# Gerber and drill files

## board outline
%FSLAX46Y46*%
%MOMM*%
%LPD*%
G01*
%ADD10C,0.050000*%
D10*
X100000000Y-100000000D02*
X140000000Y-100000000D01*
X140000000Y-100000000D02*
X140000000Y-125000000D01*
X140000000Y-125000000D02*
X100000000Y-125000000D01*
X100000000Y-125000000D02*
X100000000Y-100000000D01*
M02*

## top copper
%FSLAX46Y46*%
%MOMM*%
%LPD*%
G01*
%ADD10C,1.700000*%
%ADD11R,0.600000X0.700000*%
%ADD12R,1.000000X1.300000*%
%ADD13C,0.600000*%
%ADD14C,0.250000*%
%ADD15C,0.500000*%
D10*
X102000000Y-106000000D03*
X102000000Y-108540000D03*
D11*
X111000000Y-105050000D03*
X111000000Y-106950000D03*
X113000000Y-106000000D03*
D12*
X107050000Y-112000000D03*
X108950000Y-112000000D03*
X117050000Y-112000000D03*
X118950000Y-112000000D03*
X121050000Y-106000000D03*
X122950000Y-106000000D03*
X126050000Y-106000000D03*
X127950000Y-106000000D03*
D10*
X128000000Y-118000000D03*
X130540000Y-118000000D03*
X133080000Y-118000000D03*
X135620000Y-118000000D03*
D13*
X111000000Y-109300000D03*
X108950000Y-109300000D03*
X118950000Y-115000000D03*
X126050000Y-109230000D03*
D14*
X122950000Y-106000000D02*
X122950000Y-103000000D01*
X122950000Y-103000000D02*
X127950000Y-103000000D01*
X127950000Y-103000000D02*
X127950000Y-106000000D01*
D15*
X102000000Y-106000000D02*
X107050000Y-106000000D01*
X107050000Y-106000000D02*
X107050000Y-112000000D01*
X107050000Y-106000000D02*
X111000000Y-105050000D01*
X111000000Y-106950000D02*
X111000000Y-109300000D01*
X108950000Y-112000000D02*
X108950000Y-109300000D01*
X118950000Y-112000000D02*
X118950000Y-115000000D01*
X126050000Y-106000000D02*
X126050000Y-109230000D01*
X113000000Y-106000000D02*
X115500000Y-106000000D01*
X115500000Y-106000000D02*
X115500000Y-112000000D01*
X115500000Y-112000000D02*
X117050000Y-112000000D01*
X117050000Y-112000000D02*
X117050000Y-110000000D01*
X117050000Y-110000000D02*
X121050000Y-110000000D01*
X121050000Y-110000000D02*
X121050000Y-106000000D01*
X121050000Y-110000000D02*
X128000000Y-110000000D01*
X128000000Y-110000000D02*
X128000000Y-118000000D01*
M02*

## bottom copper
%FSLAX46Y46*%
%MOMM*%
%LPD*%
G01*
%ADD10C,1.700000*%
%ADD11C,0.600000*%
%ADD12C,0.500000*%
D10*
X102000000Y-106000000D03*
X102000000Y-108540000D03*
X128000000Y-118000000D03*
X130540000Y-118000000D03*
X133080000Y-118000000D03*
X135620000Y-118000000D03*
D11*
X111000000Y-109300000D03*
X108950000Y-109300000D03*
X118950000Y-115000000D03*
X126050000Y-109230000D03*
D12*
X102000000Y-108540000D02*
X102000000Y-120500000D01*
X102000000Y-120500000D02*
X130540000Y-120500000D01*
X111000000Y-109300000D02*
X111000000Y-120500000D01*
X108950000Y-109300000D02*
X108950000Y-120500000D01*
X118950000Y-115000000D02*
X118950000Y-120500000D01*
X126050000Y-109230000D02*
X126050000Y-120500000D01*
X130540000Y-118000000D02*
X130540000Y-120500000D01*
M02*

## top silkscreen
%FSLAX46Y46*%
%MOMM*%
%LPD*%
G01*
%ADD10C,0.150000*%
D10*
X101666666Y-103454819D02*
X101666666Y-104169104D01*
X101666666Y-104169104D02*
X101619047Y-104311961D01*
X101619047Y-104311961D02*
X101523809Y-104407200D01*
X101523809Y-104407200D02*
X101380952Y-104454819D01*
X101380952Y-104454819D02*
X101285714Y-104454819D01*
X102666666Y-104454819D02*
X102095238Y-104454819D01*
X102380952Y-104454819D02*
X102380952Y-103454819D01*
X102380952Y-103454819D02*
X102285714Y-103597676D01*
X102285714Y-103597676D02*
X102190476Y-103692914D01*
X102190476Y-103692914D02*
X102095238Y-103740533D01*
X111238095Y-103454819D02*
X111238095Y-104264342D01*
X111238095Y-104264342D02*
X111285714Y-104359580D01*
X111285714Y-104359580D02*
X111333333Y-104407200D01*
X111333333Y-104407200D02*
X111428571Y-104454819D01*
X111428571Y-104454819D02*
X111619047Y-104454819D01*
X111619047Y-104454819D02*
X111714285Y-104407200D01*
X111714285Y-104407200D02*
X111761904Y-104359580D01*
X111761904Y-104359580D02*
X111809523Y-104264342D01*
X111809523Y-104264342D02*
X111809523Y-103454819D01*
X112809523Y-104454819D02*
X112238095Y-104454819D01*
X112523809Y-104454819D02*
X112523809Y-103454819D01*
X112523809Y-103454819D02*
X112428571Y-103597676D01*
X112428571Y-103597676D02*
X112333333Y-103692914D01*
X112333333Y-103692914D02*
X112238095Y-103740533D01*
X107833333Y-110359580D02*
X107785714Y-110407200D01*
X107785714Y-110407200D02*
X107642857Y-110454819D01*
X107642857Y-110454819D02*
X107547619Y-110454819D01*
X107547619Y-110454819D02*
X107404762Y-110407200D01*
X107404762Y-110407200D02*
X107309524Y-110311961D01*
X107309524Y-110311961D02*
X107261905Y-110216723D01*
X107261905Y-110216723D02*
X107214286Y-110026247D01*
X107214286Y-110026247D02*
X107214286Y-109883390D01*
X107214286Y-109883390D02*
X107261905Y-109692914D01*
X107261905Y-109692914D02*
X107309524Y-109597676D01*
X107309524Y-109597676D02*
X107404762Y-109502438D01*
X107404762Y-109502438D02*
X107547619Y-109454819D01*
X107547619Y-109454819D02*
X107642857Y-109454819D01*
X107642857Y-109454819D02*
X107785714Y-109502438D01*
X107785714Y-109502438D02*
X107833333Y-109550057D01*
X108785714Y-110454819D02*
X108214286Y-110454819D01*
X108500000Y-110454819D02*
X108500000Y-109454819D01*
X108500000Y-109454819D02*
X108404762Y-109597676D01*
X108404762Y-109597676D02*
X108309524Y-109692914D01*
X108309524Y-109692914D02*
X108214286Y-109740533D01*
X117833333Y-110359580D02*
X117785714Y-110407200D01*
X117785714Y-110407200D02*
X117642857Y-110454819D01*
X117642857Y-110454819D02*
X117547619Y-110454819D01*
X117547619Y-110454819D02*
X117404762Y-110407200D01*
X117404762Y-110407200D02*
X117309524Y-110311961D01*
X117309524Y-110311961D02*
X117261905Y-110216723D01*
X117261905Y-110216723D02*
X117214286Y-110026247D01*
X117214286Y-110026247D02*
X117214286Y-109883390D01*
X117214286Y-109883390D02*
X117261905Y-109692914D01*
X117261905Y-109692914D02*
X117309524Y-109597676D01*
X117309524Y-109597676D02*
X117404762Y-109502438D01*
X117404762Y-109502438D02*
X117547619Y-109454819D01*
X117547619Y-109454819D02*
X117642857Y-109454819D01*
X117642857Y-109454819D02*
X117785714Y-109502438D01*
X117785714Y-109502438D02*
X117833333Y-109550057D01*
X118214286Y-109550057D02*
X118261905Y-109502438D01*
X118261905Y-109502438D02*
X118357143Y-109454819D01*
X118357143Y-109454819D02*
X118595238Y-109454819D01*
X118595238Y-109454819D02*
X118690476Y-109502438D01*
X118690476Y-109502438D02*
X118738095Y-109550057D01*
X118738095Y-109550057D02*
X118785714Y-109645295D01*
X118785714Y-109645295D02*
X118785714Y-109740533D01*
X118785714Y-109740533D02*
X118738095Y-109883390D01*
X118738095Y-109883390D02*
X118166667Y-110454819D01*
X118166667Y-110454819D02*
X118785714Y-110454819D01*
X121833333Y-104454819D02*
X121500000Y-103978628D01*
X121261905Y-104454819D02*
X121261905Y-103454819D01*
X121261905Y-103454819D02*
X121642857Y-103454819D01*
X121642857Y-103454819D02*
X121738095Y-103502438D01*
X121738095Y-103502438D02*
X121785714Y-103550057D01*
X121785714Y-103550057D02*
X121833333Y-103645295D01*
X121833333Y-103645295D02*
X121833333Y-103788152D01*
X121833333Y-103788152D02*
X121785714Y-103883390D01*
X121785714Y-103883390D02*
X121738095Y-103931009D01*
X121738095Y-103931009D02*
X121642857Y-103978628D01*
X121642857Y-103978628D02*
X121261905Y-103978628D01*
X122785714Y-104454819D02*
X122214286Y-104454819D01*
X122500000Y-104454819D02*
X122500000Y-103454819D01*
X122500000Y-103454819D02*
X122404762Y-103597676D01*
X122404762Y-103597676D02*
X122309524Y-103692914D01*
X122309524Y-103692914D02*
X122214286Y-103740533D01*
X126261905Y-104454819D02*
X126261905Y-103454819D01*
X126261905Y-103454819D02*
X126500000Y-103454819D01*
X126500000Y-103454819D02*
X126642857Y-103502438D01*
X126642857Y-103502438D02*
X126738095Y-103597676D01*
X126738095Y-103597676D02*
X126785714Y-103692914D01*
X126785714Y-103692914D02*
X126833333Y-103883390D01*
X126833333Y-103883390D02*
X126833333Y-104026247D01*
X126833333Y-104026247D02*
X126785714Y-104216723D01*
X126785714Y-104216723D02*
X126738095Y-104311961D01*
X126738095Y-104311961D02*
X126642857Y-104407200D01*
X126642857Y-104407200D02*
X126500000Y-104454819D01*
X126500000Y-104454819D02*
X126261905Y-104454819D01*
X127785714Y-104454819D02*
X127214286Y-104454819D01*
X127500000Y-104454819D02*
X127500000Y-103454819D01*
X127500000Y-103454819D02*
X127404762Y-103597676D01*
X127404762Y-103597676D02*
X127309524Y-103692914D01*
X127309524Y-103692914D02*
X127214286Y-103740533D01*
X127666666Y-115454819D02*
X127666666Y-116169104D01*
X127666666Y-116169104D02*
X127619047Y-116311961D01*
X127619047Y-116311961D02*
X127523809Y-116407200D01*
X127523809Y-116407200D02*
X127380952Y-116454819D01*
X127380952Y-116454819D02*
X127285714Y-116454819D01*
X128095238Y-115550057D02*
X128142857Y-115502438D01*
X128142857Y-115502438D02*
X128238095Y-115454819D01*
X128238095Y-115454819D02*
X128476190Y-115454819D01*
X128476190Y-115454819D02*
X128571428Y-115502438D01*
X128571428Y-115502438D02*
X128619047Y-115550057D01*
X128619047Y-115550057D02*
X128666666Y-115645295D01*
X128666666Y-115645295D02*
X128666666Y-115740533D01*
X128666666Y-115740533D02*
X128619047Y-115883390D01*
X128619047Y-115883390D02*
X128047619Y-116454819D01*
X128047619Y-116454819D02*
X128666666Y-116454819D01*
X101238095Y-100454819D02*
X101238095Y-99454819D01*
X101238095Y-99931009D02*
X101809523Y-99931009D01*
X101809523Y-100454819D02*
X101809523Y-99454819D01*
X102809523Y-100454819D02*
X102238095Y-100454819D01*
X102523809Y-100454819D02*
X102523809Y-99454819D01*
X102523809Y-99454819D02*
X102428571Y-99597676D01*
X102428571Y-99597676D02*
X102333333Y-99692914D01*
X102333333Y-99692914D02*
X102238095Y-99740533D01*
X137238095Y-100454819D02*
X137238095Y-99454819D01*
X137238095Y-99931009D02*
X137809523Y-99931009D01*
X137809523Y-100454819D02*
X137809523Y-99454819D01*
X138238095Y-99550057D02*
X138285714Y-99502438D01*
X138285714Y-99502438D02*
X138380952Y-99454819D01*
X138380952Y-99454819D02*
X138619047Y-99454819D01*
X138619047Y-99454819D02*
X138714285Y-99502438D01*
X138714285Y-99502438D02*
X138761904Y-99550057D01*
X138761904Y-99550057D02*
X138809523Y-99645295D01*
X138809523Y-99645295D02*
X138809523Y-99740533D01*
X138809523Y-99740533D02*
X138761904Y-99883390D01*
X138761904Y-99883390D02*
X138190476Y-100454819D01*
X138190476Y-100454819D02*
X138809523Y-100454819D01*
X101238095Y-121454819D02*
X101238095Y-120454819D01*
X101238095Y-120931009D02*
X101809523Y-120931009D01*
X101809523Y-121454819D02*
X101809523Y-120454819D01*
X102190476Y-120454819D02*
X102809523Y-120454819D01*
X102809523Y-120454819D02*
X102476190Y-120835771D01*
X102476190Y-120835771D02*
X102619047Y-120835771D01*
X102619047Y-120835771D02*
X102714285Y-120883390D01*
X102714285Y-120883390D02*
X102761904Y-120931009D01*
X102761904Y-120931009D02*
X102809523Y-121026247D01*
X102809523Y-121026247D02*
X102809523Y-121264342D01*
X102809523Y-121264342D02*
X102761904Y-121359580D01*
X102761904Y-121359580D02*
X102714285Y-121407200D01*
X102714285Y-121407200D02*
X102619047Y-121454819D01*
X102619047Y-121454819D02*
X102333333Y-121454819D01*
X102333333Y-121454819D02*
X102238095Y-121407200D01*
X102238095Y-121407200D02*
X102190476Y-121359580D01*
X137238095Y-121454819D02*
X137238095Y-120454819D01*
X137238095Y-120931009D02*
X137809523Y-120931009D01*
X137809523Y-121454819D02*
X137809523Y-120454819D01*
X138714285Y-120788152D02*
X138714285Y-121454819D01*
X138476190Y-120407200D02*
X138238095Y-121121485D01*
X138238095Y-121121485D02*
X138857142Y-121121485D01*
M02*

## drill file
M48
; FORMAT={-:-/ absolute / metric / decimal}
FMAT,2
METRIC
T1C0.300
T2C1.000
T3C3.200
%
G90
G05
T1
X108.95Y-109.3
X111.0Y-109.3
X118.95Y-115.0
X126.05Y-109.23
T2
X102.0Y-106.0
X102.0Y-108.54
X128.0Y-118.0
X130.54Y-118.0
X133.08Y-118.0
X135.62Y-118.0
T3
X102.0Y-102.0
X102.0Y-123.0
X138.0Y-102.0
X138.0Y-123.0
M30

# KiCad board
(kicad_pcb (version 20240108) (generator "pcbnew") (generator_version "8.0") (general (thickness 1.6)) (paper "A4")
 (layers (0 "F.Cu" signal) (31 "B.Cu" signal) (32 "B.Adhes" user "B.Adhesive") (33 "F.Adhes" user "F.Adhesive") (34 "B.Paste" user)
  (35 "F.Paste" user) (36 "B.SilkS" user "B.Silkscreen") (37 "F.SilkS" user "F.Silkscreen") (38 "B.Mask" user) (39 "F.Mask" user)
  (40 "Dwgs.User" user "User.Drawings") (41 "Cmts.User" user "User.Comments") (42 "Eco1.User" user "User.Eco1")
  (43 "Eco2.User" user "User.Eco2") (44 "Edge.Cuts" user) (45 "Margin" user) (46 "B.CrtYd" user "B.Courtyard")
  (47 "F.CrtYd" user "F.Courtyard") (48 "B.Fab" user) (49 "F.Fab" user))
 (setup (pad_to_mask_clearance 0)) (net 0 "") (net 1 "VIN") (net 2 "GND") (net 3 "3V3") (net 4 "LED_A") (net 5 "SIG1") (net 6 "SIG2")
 (gr_line (start 100 100) (end 140 100) (stroke (width 0.05) (type default)) (layer "Edge.Cuts"))
 (gr_line (start 140 100) (end 140 125) (stroke (width 0.05) (type default)) (layer "Edge.Cuts"))
 (gr_line (start 140 125) (end 100 125) (stroke (width 0.05) (type default)) (layer "Edge.Cuts"))
 (gr_line (start 100 125) (end 100 100) (stroke (width 0.05) (type default)) (layer "Edge.Cuts"))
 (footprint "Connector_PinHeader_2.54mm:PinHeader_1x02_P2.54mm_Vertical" (layer "F.Cu") (at 102 106)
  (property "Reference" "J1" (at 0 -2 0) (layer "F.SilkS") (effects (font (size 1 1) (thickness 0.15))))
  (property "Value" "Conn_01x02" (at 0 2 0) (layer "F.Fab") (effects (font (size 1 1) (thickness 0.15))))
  (pad "1" thru_hole circle (at 0 0) (size 1.7 1.7) (drill 1) (layers "*.Cu" "*.Mask") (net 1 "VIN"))
  (pad "2" thru_hole circle (at 0 2.54) (size 1.7 1.7) (drill 1) (layers "*.Cu" "*.Mask") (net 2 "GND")))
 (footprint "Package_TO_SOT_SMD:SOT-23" (layer "F.Cu") (at 112 106)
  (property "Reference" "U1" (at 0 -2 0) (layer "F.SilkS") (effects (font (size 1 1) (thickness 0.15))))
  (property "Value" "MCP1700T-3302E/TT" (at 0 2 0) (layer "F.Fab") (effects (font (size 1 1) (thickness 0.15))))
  (pad "1" smd rect (at -1 -0.95) (size 0.6 0.7) (layers "F.Cu" "F.Paste" "F.Mask") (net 1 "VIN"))
  (pad "2" smd rect (at -1 0.95) (size 0.6 0.7) (layers "F.Cu" "F.Paste" "F.Mask") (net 2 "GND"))
  (pad "3" smd rect (at 1 0) (size 0.6 0.7) (layers "F.Cu" "F.Paste" "F.Mask") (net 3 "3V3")))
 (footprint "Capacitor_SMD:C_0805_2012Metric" (layer "F.Cu") (at 108 112)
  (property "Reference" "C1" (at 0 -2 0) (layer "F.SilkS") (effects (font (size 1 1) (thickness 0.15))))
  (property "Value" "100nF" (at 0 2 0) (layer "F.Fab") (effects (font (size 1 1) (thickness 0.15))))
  (pad "1" smd rect (at -0.95 0) (size 1 1.3) (layers "F.Cu" "F.Paste" "F.Mask") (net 1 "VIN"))
  (pad "2" smd rect (at 0.95 0) (size 1 1.3) (layers "F.Cu" "F.Paste" "F.Mask") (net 2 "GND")))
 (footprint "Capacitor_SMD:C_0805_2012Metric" (layer "F.Cu") (at 118 112)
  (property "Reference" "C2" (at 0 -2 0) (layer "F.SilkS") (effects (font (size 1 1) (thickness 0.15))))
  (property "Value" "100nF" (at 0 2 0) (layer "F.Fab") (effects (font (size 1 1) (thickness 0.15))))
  (pad "1" smd rect (at -0.95 0) (size 1 1.3) (layers "F.Cu" "F.Paste" "F.Mask") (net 3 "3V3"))
  (pad "2" smd rect (at 0.95 0) (size 1 1.3) (layers "F.Cu" "F.Paste" "F.Mask") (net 2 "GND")))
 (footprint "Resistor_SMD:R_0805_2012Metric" (layer "F.Cu") (at 122 106)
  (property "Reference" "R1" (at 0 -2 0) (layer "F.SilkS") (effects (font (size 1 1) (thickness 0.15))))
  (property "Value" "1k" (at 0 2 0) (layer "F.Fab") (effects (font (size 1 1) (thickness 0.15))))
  (pad "1" smd rect (at -0.95 0) (size 1 1.3) (layers "F.Cu" "F.Paste" "F.Mask") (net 3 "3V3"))
  (pad "2" smd rect (at 0.95 0) (size 1 1.3) (layers "F.Cu" "F.Paste" "F.Mask") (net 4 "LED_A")))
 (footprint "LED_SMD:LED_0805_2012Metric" (layer "F.Cu") (at 127 106)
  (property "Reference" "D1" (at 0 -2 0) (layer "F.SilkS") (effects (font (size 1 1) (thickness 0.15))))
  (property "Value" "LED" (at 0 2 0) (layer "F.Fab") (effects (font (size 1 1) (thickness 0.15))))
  (pad "1" smd rect (at -0.95 0) (size 1 1.3) (layers "F.Cu" "F.Paste" "F.Mask") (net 2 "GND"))
  (pad "2" smd rect (at 0.95 0) (size 1 1.3) (layers "F.Cu" "F.Paste" "F.Mask") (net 4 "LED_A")))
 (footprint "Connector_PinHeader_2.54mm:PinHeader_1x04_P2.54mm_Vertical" (layer "F.Cu") (at 128 118)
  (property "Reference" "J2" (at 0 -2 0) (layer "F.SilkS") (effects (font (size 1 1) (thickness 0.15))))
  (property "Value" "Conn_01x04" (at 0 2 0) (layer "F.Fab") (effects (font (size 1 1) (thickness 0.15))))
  (pad "1" thru_hole circle (at 0 0) (size 1.7 1.7) (drill 1) (layers "*.Cu" "*.Mask") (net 3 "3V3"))
  (pad "2" thru_hole circle (at 2.54 0) (size 1.7 1.7) (drill 1) (layers "*.Cu" "*.Mask") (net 2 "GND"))
  (pad "3" thru_hole circle (at 5.08 0) (size 1.7 1.7) (drill 1) (layers "*.Cu" "*.Mask") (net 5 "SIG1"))
  (pad "4" thru_hole circle (at 7.62 0) (size 1.7 1.7) (drill 1) (layers "*.Cu" "*.Mask") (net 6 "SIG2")))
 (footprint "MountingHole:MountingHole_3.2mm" (layer "F.Cu") (at 102 102)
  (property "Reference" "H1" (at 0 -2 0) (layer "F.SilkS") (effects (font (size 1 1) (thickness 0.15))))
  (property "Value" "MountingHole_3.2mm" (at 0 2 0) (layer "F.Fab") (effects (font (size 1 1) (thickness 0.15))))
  (pad "1" np_thru_hole circle (at 0 0) (size 3.2 3.2) (drill 3.2) (layers "*.Cu" "*.Mask")))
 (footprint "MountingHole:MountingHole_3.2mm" (layer "F.Cu") (at 138 102)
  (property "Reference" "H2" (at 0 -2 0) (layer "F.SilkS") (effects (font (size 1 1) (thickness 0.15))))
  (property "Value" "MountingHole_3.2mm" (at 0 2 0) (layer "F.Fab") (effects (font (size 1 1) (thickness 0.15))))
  (pad "1" np_thru_hole circle (at 0 0) (size 3.2 3.2) (drill 3.2) (layers "*.Cu" "*.Mask")))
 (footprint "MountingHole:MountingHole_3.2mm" (layer "F.Cu") (at 102 123)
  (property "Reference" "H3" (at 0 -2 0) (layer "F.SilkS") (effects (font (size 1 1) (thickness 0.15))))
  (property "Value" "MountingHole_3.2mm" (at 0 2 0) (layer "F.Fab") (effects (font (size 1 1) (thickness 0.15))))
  (pad "1" np_thru_hole circle (at 0 0) (size 3.2 3.2) (drill 3.2) (layers "*.Cu" "*.Mask")))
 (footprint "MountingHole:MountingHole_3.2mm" (layer "F.Cu") (at 138 123)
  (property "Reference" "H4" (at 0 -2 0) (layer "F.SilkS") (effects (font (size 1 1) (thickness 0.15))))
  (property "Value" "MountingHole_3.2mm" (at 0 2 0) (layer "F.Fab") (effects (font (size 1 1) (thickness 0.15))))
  (pad "1" np_thru_hole circle (at 0 0) (size 3.2 3.2) (drill 3.2) (layers "*.Cu" "*.Mask")))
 (segment (start 122.95 106) (end 122.95 103) (width 0.25) (layer "F.Cu") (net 4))
 (segment (start 122.95 103) (end 127.95 103) (width 0.25) (layer "F.Cu") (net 4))
 (segment (start 127.95 103) (end 127.95 106) (width 0.25) (layer "F.Cu") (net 4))
 (segment (start 102 106) (end 107.05 106) (width 0.5) (layer "F.Cu") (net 1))
 (segment (start 107.05 106) (end 107.05 112) (width 0.5) (layer "F.Cu") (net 1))
 (segment (start 107.05 106) (end 111 105.05) (width 0.5) (layer "F.Cu") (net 1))
 (segment (start 111 106.95) (end 111 109.3) (width 0.5) (layer "F.Cu") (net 2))
 (segment (start 108.95 112) (end 108.95 109.3) (width 0.5) (layer "F.Cu") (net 2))
 (segment (start 118.95 112) (end 118.95 115) (width 0.5) (layer "F.Cu") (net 2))
 (segment (start 126.05 106) (end 126.05 109.23) (width 0.5) (layer "F.Cu") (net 2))
 (segment (start 113 106) (end 115.5 106) (width 0.5) (layer "F.Cu") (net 3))
 (segment (start 115.5 106) (end 115.5 112) (width 0.5) (layer "F.Cu") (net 3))
 (segment (start 115.5 112) (end 117.05 112) (width 0.5) (layer "F.Cu") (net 3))
 (segment (start 117.05 112) (end 117.05 110) (width 0.5) (layer "F.Cu") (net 3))
 (segment (start 117.05 110) (end 121.05 110) (width 0.5) (layer "F.Cu") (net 3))
 (segment (start 121.05 110) (end 121.05 106) (width 0.5) (layer "F.Cu") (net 3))
 (segment (start 121.05 110) (end 128 110) (width 0.5) (layer "F.Cu") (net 3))
 (segment (start 128 110) (end 128 118) (width 0.5) (layer "F.Cu") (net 3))
 (segment (start 102 108.54) (end 102 120.5) (width 0.5) (layer "B.Cu") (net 2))
 (segment (start 102 120.5) (end 130.54 120.5) (width 0.5) (layer "B.Cu") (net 2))
 (segment (start 111 109.3) (end 111 120.5) (width 0.5) (layer "B.Cu") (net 2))
 (segment (start 108.95 109.3) (end 108.95 120.5) (width 0.5) (layer "B.Cu") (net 2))
 (segment (start 118.95 115) (end 118.95 120.5) (width 0.5) (layer "B.Cu") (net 2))
 (segment (start 126.05 109.23) (end 126.05 120.5) (width 0.5) (layer "B.Cu") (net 2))
 (segment (start 130.54 118) (end 130.54 120.5) (width 0.5) (layer "B.Cu") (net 2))
 (via (at 111 109.3) (size 0.6) (drill 0.3) (layers "F.Cu" "B.Cu") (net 2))
 (via (at 108.95 109.3) (size 0.6) (drill 0.3) (layers "F.Cu" "B.Cu") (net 2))
 (via (at 118.95 115) (size 0.6) (drill 0.3) (layers "F.Cu" "B.Cu") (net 2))
 (via (at 126.05 109.23) (size 0.6) (drill 0.3) (layers "F.Cu" "B.Cu") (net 2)))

